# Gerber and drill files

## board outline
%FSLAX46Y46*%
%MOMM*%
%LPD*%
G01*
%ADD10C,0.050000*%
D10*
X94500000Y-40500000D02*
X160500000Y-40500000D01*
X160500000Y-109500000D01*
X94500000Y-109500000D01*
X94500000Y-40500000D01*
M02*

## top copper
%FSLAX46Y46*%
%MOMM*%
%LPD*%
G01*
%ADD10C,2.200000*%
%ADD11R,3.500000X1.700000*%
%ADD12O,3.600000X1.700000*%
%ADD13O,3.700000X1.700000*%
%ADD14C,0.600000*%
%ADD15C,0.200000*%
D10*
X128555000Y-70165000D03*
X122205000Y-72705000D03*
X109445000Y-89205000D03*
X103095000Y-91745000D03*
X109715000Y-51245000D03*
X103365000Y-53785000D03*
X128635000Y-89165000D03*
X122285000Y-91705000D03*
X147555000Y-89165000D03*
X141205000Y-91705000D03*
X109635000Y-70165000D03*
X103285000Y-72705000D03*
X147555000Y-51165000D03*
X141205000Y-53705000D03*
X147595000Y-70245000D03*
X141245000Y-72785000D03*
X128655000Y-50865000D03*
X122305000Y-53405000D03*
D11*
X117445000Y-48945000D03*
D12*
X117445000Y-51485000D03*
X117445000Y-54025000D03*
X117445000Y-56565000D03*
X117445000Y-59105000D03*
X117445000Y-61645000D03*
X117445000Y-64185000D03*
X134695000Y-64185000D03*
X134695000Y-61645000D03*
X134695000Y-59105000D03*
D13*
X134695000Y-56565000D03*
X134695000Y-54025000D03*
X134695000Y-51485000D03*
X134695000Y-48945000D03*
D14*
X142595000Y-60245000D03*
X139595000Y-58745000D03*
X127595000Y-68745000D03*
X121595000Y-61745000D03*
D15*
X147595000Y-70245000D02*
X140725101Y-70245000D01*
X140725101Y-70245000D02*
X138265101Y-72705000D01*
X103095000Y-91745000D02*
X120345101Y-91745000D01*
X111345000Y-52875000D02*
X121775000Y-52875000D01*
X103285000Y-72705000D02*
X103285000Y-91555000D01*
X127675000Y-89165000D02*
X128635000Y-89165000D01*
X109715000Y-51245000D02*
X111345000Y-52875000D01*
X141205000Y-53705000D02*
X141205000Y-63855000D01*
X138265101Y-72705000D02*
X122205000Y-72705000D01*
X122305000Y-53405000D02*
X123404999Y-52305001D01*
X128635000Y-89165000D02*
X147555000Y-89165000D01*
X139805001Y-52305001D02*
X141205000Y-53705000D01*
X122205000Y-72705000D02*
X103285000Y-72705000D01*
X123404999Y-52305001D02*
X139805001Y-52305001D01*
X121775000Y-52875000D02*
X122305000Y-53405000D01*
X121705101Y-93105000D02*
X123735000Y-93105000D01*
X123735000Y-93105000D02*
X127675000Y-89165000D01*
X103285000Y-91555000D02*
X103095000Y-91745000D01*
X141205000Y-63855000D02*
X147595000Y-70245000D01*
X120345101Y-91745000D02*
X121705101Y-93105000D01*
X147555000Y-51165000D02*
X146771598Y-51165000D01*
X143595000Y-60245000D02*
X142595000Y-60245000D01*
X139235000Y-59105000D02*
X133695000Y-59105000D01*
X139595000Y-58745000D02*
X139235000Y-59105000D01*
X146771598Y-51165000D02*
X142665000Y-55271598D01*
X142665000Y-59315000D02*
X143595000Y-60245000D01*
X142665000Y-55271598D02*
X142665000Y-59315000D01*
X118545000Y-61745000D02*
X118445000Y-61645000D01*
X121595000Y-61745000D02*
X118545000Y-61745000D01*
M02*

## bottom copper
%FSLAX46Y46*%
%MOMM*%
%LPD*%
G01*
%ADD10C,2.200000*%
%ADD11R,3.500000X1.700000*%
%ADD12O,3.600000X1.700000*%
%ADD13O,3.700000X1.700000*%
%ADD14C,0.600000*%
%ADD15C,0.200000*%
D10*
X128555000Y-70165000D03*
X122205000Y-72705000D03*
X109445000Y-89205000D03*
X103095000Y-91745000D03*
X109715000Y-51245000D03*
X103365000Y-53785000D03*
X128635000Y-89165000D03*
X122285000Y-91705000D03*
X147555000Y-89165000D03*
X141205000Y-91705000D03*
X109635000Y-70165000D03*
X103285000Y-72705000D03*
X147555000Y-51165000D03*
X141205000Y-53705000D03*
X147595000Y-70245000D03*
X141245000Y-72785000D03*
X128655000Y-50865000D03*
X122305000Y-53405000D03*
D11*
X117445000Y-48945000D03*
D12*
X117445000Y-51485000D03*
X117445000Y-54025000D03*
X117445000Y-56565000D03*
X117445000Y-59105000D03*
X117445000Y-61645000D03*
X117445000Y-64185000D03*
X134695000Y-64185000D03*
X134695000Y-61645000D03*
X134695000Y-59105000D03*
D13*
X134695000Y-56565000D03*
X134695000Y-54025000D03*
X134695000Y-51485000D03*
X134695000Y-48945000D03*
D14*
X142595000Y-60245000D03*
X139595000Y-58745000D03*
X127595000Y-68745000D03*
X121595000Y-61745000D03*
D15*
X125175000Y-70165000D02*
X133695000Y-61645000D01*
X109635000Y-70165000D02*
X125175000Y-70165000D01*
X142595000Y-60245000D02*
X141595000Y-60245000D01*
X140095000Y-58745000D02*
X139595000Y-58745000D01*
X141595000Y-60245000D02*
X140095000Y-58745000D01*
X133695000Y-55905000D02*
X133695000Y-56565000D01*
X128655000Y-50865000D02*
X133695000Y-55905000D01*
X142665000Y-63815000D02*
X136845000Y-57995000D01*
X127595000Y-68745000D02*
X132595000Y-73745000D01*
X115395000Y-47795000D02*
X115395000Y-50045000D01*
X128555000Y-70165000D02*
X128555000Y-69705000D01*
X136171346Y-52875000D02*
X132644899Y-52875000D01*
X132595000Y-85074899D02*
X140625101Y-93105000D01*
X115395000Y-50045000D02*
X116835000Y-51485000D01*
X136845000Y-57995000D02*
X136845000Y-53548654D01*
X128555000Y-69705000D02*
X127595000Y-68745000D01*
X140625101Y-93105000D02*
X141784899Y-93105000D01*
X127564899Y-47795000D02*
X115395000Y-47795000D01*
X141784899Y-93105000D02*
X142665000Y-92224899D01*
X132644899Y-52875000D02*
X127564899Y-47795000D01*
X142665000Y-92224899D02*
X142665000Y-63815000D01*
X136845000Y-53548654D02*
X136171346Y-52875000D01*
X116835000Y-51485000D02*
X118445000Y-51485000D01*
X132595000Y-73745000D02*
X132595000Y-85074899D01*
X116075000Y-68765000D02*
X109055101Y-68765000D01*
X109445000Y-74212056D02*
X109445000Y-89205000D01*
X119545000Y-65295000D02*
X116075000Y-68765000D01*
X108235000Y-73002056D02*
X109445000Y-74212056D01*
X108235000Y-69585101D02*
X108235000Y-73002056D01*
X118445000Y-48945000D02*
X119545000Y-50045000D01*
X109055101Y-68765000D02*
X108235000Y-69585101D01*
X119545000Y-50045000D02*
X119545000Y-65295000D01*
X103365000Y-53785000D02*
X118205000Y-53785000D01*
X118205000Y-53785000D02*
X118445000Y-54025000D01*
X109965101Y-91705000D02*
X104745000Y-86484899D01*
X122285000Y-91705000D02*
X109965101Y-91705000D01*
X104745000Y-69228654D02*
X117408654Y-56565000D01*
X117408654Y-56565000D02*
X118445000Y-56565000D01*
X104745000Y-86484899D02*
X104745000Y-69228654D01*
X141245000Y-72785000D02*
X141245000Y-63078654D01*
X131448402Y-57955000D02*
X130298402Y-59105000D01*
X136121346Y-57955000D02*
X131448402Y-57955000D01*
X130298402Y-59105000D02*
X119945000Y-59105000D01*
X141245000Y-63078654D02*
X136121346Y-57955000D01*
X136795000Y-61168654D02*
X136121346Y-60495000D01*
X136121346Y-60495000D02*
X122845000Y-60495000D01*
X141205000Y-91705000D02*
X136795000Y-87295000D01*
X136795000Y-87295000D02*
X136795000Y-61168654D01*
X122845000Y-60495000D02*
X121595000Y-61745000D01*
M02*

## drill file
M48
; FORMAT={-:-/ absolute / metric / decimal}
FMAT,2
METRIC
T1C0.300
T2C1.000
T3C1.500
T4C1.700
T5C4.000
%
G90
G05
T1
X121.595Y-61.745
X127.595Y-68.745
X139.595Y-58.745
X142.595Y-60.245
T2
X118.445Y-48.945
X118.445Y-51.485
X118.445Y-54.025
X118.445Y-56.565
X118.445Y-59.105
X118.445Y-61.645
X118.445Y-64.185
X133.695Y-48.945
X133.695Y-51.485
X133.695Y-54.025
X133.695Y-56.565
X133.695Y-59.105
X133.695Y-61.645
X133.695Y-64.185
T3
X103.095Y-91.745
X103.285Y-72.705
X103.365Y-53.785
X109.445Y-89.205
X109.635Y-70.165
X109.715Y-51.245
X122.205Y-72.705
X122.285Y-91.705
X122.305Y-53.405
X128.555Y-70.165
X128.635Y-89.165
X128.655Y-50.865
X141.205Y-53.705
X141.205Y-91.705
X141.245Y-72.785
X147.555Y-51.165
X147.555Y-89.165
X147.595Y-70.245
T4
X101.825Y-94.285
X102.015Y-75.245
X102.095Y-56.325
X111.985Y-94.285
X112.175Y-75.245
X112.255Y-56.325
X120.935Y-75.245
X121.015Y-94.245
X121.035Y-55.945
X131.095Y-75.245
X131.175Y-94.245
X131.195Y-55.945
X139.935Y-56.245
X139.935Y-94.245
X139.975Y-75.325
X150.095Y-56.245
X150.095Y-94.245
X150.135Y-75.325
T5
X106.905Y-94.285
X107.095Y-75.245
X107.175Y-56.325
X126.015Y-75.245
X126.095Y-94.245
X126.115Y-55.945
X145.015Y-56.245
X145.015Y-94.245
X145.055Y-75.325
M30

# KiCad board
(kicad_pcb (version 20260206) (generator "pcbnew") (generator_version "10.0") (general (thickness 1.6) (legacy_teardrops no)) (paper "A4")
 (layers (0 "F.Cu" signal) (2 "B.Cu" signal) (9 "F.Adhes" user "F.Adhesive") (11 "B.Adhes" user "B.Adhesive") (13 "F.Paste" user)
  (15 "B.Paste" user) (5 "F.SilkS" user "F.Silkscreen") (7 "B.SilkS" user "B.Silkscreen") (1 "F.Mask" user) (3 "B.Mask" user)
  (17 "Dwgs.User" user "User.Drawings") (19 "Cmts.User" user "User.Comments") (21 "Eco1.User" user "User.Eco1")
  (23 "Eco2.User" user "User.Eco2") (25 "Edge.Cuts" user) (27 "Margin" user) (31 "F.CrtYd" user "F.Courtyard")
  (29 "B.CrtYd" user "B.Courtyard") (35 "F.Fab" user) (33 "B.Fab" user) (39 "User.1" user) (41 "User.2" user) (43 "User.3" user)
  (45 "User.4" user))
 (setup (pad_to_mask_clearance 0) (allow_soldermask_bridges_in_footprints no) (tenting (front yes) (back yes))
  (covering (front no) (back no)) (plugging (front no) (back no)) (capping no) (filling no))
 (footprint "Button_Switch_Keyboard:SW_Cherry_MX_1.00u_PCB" (layer "F.Cu") (at 128.555 70.165)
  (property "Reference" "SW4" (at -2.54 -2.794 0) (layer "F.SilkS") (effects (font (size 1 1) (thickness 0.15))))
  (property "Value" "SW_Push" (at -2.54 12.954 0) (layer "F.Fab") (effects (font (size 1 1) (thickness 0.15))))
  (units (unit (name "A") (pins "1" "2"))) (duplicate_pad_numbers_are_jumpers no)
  (pad "" np_thru_hole circle (at -7.62 5.08) (size 1.7 1.7) (drill 1.7) (layers "*.Cu" "*.Mask"))
  (pad "" np_thru_hole circle (at -2.54 5.08) (size 4 4) (drill 4) (layers "*.Cu" "*.Mask"))
  (pad "" np_thru_hole circle (at 2.54 5.08) (size 1.7 1.7) (drill 1.7) (layers "*.Cu" "*.Mask"))
  (pad "1" thru_hole circle (at 0 0) (size 2.2 2.2) (drill 1.5) (layers "*.Cu" "*.Mask") (remove_unused_layers no)
   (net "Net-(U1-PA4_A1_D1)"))
  (pad "2" thru_hole circle (at -6.35 2.54) (size 2.2 2.2) (drill 1.5) (layers "*.Cu" "*.Mask") (remove_unused_layers no) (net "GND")))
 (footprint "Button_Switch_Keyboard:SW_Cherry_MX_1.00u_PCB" (layer "F.Cu") (at 109.445 89.205)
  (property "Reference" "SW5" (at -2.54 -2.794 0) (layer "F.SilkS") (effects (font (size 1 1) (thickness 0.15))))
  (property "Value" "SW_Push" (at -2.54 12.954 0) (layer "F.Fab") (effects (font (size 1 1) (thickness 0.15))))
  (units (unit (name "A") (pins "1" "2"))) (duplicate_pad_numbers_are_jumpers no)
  (pad "" np_thru_hole circle (at -7.62 5.08) (size 1.7 1.7) (drill 1.7) (layers "*.Cu" "*.Mask"))
  (pad "" np_thru_hole circle (at -2.54 5.08) (size 4 4) (drill 4) (layers "*.Cu" "*.Mask"))
  (pad "" np_thru_hole circle (at 2.54 5.08) (size 1.7 1.7) (drill 1.7) (layers "*.Cu" "*.Mask"))
  (pad "1" thru_hole circle (at 0 0) (size 2.2 2.2) (drill 1.5) (layers "*.Cu" "*.Mask") (remove_unused_layers no)
   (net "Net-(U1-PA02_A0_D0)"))
  (pad "2" thru_hole circle (at -6.35 2.54) (size 2.2 2.2) (drill 1.5) (layers "*.Cu" "*.Mask") (remove_unused_layers no) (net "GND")))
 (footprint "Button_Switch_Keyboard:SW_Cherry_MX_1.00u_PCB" (layer "F.Cu") (at 109.715 51.245)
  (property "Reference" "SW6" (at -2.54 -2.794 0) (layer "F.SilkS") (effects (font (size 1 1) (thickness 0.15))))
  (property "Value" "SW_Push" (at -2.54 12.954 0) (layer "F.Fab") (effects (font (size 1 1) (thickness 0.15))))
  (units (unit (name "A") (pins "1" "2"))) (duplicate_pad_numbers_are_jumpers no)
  (pad "" np_thru_hole circle (at -7.62 5.08) (size 1.7 1.7) (drill 1.7) (layers "*.Cu" "*.Mask"))
  (pad "" np_thru_hole circle (at -2.54 5.08) (size 4 4) (drill 4) (layers "*.Cu" "*.Mask"))
  (pad "" np_thru_hole circle (at 2.54 5.08) (size 1.7 1.7) (drill 1.7) (layers "*.Cu" "*.Mask"))
  (pad "1" thru_hole circle (at 0 0) (size 2.2 2.2) (drill 1.5) (layers "*.Cu" "*.Mask") (remove_unused_layers no) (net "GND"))
  (pad "2" thru_hole circle (at -6.35 2.54) (size 2.2 2.2) (drill 1.5) (layers "*.Cu" "*.Mask") (remove_unused_layers no)
   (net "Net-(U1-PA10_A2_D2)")))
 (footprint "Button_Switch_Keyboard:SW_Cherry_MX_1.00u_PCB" (layer "F.Cu") (at 128.635 89.165)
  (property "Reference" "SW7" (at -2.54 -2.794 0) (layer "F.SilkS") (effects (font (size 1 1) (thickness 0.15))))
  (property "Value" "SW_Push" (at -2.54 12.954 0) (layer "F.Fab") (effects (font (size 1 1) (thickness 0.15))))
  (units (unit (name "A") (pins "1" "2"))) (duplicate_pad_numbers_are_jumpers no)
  (pad "" np_thru_hole circle (at -7.62 5.08) (size 1.7 1.7) (drill 1.7) (layers "*.Cu" "*.Mask"))
  (pad "" np_thru_hole circle (at -2.54 5.08) (size 4 4) (drill 4) (layers "*.Cu" "*.Mask"))
  (pad "" np_thru_hole circle (at 2.54 5.08) (size 1.7 1.7) (drill 1.7) (layers "*.Cu" "*.Mask"))
  (pad "1" thru_hole circle (at 0 0) (size 2.2 2.2) (drill 1.5) (layers "*.Cu" "*.Mask") (remove_unused_layers no) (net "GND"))
  (pad "2" thru_hole circle (at -6.35 2.54) (size 2.2 2.2) (drill 1.5) (layers "*.Cu" "*.Mask") (remove_unused_layers no)
   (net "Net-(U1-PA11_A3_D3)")))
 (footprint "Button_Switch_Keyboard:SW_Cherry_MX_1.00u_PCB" (layer "F.Cu") (at 147.555 89.165)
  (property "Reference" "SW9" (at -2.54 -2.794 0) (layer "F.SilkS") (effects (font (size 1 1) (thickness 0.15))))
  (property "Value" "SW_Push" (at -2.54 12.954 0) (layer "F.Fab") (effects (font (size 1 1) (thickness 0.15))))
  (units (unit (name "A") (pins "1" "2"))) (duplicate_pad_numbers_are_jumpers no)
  (pad "" np_thru_hole circle (at -7.62 5.08) (size 1.7 1.7) (drill 1.7) (layers "*.Cu" "*.Mask"))
  (pad "" np_thru_hole circle (at -2.54 5.08) (size 4 4) (drill 4) (layers "*.Cu" "*.Mask"))
  (pad "" np_thru_hole circle (at 2.54 5.08) (size 1.7 1.7) (drill 1.7) (layers "*.Cu" "*.Mask"))
  (pad "1" thru_hole circle (at 0 0) (size 2.2 2.2) (drill 1.5) (layers "*.Cu" "*.Mask") (remove_unused_layers no) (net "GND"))
  (pad "2" thru_hole circle (at -6.35 2.54) (size 2.2 2.2) (drill 1.5) (layers "*.Cu" "*.Mask") (remove_unused_layers no)
   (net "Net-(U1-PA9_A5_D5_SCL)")))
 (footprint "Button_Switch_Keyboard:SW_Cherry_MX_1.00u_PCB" (layer "F.Cu") (at 109.635 70.165)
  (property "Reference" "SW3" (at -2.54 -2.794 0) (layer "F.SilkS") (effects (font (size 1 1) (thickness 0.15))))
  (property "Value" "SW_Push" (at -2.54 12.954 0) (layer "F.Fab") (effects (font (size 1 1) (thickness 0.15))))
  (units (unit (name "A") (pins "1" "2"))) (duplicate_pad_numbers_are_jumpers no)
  (pad "" np_thru_hole circle (at -7.62 5.08) (size 1.7 1.7) (drill 1.7) (layers "*.Cu" "*.Mask"))
  (pad "" np_thru_hole circle (at -2.54 5.08) (size 4 4) (drill 4) (layers "*.Cu" "*.Mask"))
  (pad "" np_thru_hole circle (at 2.54 5.08) (size 1.7 1.7) (drill 1.7) (layers "*.Cu" "*.Mask"))
  (pad "1" thru_hole circle (at 0 0) (size 2.2 2.2) (drill 1.5) (layers "*.Cu" "*.Mask") (remove_unused_layers no)
   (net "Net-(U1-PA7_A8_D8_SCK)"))
  (pad "2" thru_hole circle (at -6.35 2.54) (size 2.2 2.2) (drill 1.5) (layers "*.Cu" "*.Mask") (remove_unused_layers no) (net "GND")))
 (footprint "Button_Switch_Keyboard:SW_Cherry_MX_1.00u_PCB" (layer "F.Cu") (at 147.555 51.165)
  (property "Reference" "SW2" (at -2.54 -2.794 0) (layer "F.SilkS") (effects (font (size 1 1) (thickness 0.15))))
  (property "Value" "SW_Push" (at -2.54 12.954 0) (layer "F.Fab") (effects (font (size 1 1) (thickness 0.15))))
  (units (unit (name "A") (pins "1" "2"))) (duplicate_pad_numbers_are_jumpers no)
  (pad "" np_thru_hole circle (at -7.62 5.08) (size 1.7 1.7) (drill 1.7) (layers "*.Cu" "*.Mask"))
  (pad "" np_thru_hole circle (at -2.54 5.08) (size 4 4) (drill 4) (layers "*.Cu" "*.Mask"))
  (pad "" np_thru_hole circle (at 2.54 5.08) (size 1.7 1.7) (drill 1.7) (layers "*.Cu" "*.Mask"))
  (pad "1" thru_hole circle (at 0 0) (size 2.2 2.2) (drill 1.5) (layers "*.Cu" "*.Mask") (remove_unused_layers no)
   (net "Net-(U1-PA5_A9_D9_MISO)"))
  (pad "2" thru_hole circle (at -6.35 2.54) (size 2.2 2.2) (drill 1.5) (layers "*.Cu" "*.Mask") (remove_unused_layers no) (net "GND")))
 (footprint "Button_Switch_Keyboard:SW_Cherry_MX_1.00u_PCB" (layer "F.Cu") (at 147.595 70.245)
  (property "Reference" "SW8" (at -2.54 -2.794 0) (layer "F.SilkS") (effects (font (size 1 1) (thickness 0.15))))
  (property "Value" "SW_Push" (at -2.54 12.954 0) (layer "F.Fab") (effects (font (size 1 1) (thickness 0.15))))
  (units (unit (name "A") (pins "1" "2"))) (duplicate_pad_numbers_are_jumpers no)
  (pad "" np_thru_hole circle (at -7.62 5.08) (size 1.7 1.7) (drill 1.7) (layers "*.Cu" "*.Mask"))
  (pad "" np_thru_hole circle (at -2.54 5.08) (size 4 4) (drill 4) (layers "*.Cu" "*.Mask"))
  (pad "" np_thru_hole circle (at 2.54 5.08) (size 1.7 1.7) (drill 1.7) (layers "*.Cu" "*.Mask"))
  (pad "1" thru_hole circle (at 0 0) (size 2.2 2.2) (drill 1.5) (layers "*.Cu" "*.Mask") (remove_unused_layers no) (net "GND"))
  (pad "2" thru_hole circle (at -6.35 2.54) (size 2.2 2.2) (drill 1.5) (layers "*.Cu" "*.Mask") (remove_unused_layers no)
   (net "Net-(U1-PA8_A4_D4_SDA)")))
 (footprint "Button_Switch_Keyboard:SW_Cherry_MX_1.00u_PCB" (layer "F.Cu") (at 128.655 50.865)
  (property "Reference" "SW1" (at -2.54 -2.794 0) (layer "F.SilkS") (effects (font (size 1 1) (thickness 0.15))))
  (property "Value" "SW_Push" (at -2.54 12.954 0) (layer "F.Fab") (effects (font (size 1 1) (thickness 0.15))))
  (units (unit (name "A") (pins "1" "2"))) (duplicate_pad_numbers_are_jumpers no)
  (pad "" np_thru_hole circle (at -7.62 5.08) (size 1.7 1.7) (drill 1.7) (layers "*.Cu" "*.Mask"))
  (pad "" np_thru_hole circle (at -2.54 5.08) (size 4 4) (drill 4) (layers "*.Cu" "*.Mask"))
  (pad "" np_thru_hole circle (at 2.54 5.08) (size 1.7 1.7) (drill 1.7) (layers "*.Cu" "*.Mask"))
  (pad "1" thru_hole circle (at 0 0) (size 2.2 2.2) (drill 1.5) (layers "*.Cu" "*.Mask") (remove_unused_layers no)
   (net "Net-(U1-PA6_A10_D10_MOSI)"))
  (pad "2" thru_hole circle (at -6.35 2.54) (size 2.2 2.2) (drill 1.5) (layers "*.Cu" "*.Mask") (remove_unused_layers no) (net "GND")))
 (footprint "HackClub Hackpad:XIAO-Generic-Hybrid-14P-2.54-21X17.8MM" (layer "F.Cu") (at 126.07 56.565)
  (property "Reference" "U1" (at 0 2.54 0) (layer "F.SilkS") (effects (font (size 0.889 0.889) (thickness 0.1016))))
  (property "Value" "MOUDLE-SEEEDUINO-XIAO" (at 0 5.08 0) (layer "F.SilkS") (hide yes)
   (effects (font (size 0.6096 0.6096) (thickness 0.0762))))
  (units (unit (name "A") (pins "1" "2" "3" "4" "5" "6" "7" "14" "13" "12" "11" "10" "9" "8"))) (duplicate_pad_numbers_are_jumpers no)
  (pad "1" thru_hole rect (at -7.625 -7.62) (size 3.5 1.7) (drill 1 (offset -1 0)) (layers "*.Cu" "*.Mask") (remove_unused_layers no)
   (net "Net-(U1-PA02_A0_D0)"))
  (pad "2" thru_hole oval (at -7.625 -5.08) (size 3.6 1.7) (drill 1 (offset -1 0)) (layers "*.Cu" "*.Mask") (remove_unused_layers no)
   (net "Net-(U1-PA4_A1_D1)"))
  (pad "3" thru_hole oval (at -7.625 -2.54) (size 3.6 1.7) (drill 1 (offset -1 0)) (layers "*.Cu" "*.Mask") (remove_unused_layers no)
   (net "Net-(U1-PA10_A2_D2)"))
  (pad "4" thru_hole oval (at -7.625 0) (size 3.6 1.7) (drill 1 (offset -1 0)) (layers "*.Cu" "*.Mask") (remove_unused_layers no)
   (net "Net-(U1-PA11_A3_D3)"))
  (pad "5" thru_hole oval (at -7.625 2.54) (size 3.6 1.7) (drill 1 (offset -1 0)) (layers "*.Cu" "*.Mask") (remove_unused_layers no)
   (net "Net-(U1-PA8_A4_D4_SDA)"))
  (pad "6" thru_hole oval (at -7.625 5.08 180) (size 3.6 1.7) (drill 1 (offset 1 0)) (layers "*.Cu" "*.Mask") (remove_unused_layers no)
   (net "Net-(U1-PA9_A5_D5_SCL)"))
  (pad "7" thru_hole oval (at -7.625 7.62) (size 3.6 1.7) (drill 1 (offset -1 0)) (layers "*.Cu" "*.Mask") (remove_unused_layers no)
   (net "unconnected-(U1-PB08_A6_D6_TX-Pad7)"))
  (pad "8" thru_hole oval (at 7.625 7.62) (size 3.6 1.7) (drill 1 (offset 1 0)) (layers "*.Cu" "*.Mask") (remove_unused_layers no)
   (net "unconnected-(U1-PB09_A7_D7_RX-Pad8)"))
  (pad "9" thru_hole oval (at 7.625 5.08) (size 3.6 1.7) (drill 1 (offset 1 0)) (layers "*.Cu" "*.Mask") (remove_unused_layers no)
   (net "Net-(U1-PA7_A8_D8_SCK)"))
  (pad "10" thru_hole oval (at 7.625 2.54) (size 3.6 1.7) (drill 1 (offset 1 0)) (layers "*.Cu" "*.Mask") (remove_unused_layers no)
   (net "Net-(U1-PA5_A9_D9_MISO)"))
  (pad "11" thru_hole oval (at 7.625 0) (size 3.7 1.7) (drill 1 (offset 1 0)) (layers "*.Cu" "*.Mask") (remove_unused_layers no)
   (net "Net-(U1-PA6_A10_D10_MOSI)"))
  (pad "12" thru_hole oval (at 7.625 -2.54) (size 3.7 1.7) (drill 1 (offset 1 0)) (layers "*.Cu" "*.Mask") (remove_unused_layers no)
   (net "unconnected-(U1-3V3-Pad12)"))
  (pad "13" thru_hole oval (at 7.625 -5.08) (size 3.7 1.7) (drill 1 (offset 1 0)) (layers "*.Cu" "*.Mask") (remove_unused_layers no)
   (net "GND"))
  (pad "14" thru_hole oval (at 7.625 -7.62) (size 3.7 1.7) (drill 1 (offset 1 0)) (layers "*.Cu" "*.Mask") (remove_unused_layers no)
   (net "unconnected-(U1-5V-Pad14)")))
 (gr_rect (start 94.5 40.5) (end 160.5 109.5) (stroke (width 0.05) (type default)) (fill no) (layer "Edge.Cuts"))
 (segment (start 125.175 70.165) (end 133.695 61.645) (width 0.2) (layer "B.Cu") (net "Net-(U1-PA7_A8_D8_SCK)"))
 (segment (start 109.635 70.165) (end 125.175 70.165) (width 0.2) (layer "B.Cu") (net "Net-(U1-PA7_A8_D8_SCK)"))
 (segment (start 147.595 70.245) (end 140.725101 70.245) (width 0.2) (layer "F.Cu") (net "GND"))
 (segment (start 140.725101 70.245) (end 138.265101 72.705) (width 0.2) (layer "F.Cu") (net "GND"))
 (segment (start 103.095 91.745) (end 120.345101 91.745) (width 0.2) (layer "F.Cu") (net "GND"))
 (segment (start 111.345 52.875) (end 121.775 52.875) (width 0.2) (layer "F.Cu") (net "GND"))
 (segment (start 103.285 72.705) (end 103.285 91.555) (width 0.2) (layer "F.Cu") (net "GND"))
 (segment (start 127.675 89.165) (end 128.635 89.165) (width 0.2) (layer "F.Cu") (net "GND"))
 (segment (start 109.715 51.245) (end 111.345 52.875) (width 0.2) (layer "F.Cu") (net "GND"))
 (segment (start 141.205 53.705) (end 141.205 63.855) (width 0.2) (layer "F.Cu") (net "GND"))
 (segment (start 138.265101 72.705) (end 122.205 72.705) (width 0.2) (layer "F.Cu") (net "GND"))
 (segment (start 122.305 53.405) (end 123.404999 52.305001) (width 0.2) (layer "F.Cu") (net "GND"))
 (segment (start 128.635 89.165) (end 147.555 89.165) (width 0.2) (layer "F.Cu") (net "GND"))
 (segment (start 139.805001 52.305001) (end 141.205 53.705) (width 0.2) (layer "F.Cu") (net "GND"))
 (segment (start 122.205 72.705) (end 103.285 72.705) (width 0.2) (layer "F.Cu") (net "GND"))
 (segment (start 123.404999 52.305001) (end 139.805001 52.305001) (width 0.2) (layer "F.Cu") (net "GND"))
 (segment (start 121.775 52.875) (end 122.305 53.405) (width 0.2) (layer "F.Cu") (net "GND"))
 (segment (start 121.705101 93.105) (end 123.735 93.105) (width 0.2) (layer "F.Cu") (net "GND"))
 (segment (start 123.735 93.105) (end 127.675 89.165) (width 0.2) (layer "F.Cu") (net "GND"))
 (segment (start 103.285 91.555) (end 103.095 91.745) (width 0.2) (layer "F.Cu") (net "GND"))
 (segment (start 141.205 63.855) (end 147.595 70.245) (width 0.2) (layer "F.Cu") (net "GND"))
 (segment (start 120.345101 91.745) (end 121.705101 93.105) (width 0.2) (layer "F.Cu") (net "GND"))
 (segment (start 147.555 51.165) (end 146.771598 51.165) (width 0.2) (layer "F.Cu") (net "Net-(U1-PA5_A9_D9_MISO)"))
 (segment (start 143.595 60.245) (end 142.595 60.245) (width 0.2) (layer "F.Cu") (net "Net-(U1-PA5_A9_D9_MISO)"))
 (segment (start 139.235 59.105) (end 133.695 59.105) (width 0.2) (layer "F.Cu") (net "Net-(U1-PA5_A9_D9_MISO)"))
 (segment (start 139.595 58.745) (end 139.235 59.105) (width 0.2) (layer "F.Cu") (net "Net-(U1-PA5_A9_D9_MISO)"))
 (segment (start 146.771598 51.165) (end 142.665 55.271598) (width 0.2) (layer "F.Cu") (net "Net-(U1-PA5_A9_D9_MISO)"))
 (segment (start 142.665 59.315) (end 143.595 60.245) (width 0.2) (layer "F.Cu") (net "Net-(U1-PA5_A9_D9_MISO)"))
 (segment (start 142.665 55.271598) (end 142.665 59.315) (width 0.2) (layer "F.Cu") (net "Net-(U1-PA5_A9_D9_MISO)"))
 (via (at 142.595 60.245) (size 0.6) (drill 0.3) (layers "F.Cu" "B.Cu") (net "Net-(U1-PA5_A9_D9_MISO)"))
 (via (at 139.595 58.745) (size 0.6) (drill 0.3) (layers "F.Cu" "B.Cu") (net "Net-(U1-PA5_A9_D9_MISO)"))
 (segment (start 142.595 60.245) (end 141.595 60.245) (width 0.2) (layer "B.Cu") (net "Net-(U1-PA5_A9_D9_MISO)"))
 (segment (start 140.095 58.745) (end 139.595 58.745) (width 0.2) (layer "B.Cu") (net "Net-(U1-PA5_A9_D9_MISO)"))
 (segment (start 141.595 60.245) (end 140.095 58.745) (width 0.2) (layer "B.Cu") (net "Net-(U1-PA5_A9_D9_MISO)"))
 (segment (start 133.695 55.905) (end 133.695 56.565) (width 0.2) (layer "B.Cu") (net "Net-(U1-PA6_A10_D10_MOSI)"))
 (segment (start 128.655 50.865) (end 133.695 55.905) (width 0.2) (layer "B.Cu") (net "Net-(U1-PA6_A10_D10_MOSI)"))
 (via (at 127.595 68.745) (size 0.6) (drill 0.3) (layers "F.Cu" "B.Cu") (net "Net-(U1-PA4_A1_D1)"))
 (segment (start 142.665 63.815) (end 136.845 57.995) (width 0.2) (layer "B.Cu") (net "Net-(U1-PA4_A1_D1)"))
 (segment (start 127.595 68.745) (end 132.595 73.745) (width 0.2) (layer "B.Cu") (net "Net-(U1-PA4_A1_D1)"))
 (segment (start 115.395 47.795) (end 115.395 50.045) (width 0.2) (layer "B.Cu") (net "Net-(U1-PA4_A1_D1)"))
 (segment (start 128.555 70.165) (end 128.555 69.705) (width 0.2) (layer "B.Cu") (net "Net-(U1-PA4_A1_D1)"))
 (segment (start 136.171346 52.875) (end 132.644899 52.875) (width 0.2) (layer "B.Cu") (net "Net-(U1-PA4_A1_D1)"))
 (segment (start 132.595 85.074899) (end 140.625101 93.105) (width 0.2) (layer "B.Cu") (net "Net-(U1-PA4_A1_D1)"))
 (segment (start 115.395 50.045) (end 116.835 51.485) (width 0.2) (layer "B.Cu") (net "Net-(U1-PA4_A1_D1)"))
 (segment (start 136.845 57.995) (end 136.845 53.548654) (width 0.2) (layer "B.Cu") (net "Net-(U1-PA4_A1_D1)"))
 (segment (start 128.555 69.705) (end 127.595 68.745) (width 0.2) (layer "B.Cu") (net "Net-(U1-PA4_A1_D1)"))
 (segment (start 140.625101 93.105) (end 141.784899 93.105) (width 0.2) (layer "B.Cu") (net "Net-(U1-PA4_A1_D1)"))
 (segment (start 127.564899 47.795) (end 115.395 47.795) (width 0.2) (layer "B.Cu") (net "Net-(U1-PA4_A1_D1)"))
 (segment (start 141.784899 93.105) (end 142.665 92.224899) (width 0.2) (layer "B.Cu") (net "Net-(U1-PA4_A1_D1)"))
 (segment (start 132.644899 52.875) (end 127.564899 47.795) (width 0.2) (layer "B.Cu") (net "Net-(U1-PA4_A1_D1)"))
 (segment (start 142.665 92.224899) (end 142.665 63.815) (width 0.2) (layer "B.Cu") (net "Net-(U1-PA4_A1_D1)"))
 (segment (start 136.845 53.548654) (end 136.171346 52.875) (width 0.2) (layer "B.Cu") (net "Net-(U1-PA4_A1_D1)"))
 (segment (start 116.835 51.485) (end 118.445 51.485) (width 0.2) (layer "B.Cu") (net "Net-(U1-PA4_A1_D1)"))
 (segment (start 132.595 73.745) (end 132.595 85.074899) (width 0.2) (layer "B.Cu") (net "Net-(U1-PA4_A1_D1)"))
 (segment (start 116.075 68.765) (end 109.055101 68.765) (width 0.2) (layer "B.Cu") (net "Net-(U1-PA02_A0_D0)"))
 (segment (start 109.445 74.212056) (end 109.445 89.205) (width 0.2) (layer "B.Cu") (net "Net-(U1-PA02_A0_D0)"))
 (segment (start 119.545 65.295) (end 116.075 68.765) (width 0.2) (layer "B.Cu") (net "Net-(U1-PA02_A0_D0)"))
 (segment (start 108.235 73.002056) (end 109.445 74.212056) (width 0.2) (layer "B.Cu") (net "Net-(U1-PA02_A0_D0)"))
 (segment (start 108.235 69.585101) (end 108.235 73.002056) (width 0.2) (layer "B.Cu") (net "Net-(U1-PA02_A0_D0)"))
 (segment (start 118.445 48.945) (end 119.545 50.045) (width 0.2) (layer "B.Cu") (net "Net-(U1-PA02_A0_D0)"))
 (segment (start 109.055101 68.765) (end 108.235 69.585101) (width 0.2) (layer "B.Cu") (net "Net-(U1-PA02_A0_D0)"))
 (segment (start 119.545 50.045) (end 119.545 65.295) (width 0.2) (layer "B.Cu") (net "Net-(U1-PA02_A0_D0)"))
 (segment (start 103.365 53.785) (end 118.205 53.785) (width 0.2) (layer "B.Cu") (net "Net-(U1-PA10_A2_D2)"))
 (segment (start 118.205 53.785) (end 118.445 54.025) (width 0.2) (layer "B.Cu") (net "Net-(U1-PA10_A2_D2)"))
 (segment (start 109.965101 91.705) (end 104.745 86.484899) (width 0.2) (layer "B.Cu") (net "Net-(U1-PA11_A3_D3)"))
 (segment (start 122.285 91.705) (end 109.965101 91.705) (width 0.2) (layer "B.Cu") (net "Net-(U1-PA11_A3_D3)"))
 (segment (start 104.745 69.228654) (end 117.408654 56.565) (width 0.2) (layer "B.Cu") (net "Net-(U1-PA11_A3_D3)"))
 (segment (start 117.408654 56.565) (end 118.445 56.565) (width 0.2) (layer "B.Cu") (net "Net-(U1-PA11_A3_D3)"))
 (segment (start 104.745 86.484899) (end 104.745 69.228654) (width 0.2) (layer "B.Cu") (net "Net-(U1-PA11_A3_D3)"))
 (segment (start 141.245 72.785) (end 141.245 63.078654) (width 0.2) (layer "B.Cu") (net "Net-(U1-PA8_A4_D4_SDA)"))
 (segment (start 131.448402 57.955) (end 130.298402 59.105) (width 0.2) (layer "B.Cu") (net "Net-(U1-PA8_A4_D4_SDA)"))
 (segment (start 136.121346 57.955) (end 131.448402 57.955) (width 0.2) (layer "B.Cu") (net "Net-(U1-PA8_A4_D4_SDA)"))
 (segment (start 130.298402 59.105) (end 119.945 59.105) (width 0.2) (layer "B.Cu") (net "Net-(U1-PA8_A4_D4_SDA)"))
 (segment (start 141.245 63.078654) (end 136.121346 57.955) (width 0.2) (layer "B.Cu") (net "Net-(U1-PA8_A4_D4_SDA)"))
 (segment (start 118.545 61.745) (end 118.445 61.645) (width 0.2) (layer "F.Cu") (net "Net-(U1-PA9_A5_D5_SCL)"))
 (segment (start 121.595 61.745) (end 118.545 61.745) (width 0.2) (layer "F.Cu") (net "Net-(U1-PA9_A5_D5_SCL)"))
 (via (at 121.595 61.745) (size 0.6) (drill 0.3) (layers "F.Cu" "B.Cu") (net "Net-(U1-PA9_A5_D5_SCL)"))
 (segment (start 136.795 61.168654) (end 136.121346 60.495) (width 0.2) (layer "B.Cu") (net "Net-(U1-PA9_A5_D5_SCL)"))
 (segment (start 136.121346 60.495) (end 122.845 60.495) (width 0.2) (layer "B.Cu") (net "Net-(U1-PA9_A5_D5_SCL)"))
 (segment (start 141.205 91.705) (end 136.795 87.295) (width 0.2) (layer "B.Cu") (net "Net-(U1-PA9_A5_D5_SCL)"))
 (segment (start 136.795 87.295) (end 136.795 61.168654) (width 0.2) (layer "B.Cu") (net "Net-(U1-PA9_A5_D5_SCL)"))
 (segment (start 122.845 60.495) (end 121.595 61.745) (width 0.2) (layer "B.Cu") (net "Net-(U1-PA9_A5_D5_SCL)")))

